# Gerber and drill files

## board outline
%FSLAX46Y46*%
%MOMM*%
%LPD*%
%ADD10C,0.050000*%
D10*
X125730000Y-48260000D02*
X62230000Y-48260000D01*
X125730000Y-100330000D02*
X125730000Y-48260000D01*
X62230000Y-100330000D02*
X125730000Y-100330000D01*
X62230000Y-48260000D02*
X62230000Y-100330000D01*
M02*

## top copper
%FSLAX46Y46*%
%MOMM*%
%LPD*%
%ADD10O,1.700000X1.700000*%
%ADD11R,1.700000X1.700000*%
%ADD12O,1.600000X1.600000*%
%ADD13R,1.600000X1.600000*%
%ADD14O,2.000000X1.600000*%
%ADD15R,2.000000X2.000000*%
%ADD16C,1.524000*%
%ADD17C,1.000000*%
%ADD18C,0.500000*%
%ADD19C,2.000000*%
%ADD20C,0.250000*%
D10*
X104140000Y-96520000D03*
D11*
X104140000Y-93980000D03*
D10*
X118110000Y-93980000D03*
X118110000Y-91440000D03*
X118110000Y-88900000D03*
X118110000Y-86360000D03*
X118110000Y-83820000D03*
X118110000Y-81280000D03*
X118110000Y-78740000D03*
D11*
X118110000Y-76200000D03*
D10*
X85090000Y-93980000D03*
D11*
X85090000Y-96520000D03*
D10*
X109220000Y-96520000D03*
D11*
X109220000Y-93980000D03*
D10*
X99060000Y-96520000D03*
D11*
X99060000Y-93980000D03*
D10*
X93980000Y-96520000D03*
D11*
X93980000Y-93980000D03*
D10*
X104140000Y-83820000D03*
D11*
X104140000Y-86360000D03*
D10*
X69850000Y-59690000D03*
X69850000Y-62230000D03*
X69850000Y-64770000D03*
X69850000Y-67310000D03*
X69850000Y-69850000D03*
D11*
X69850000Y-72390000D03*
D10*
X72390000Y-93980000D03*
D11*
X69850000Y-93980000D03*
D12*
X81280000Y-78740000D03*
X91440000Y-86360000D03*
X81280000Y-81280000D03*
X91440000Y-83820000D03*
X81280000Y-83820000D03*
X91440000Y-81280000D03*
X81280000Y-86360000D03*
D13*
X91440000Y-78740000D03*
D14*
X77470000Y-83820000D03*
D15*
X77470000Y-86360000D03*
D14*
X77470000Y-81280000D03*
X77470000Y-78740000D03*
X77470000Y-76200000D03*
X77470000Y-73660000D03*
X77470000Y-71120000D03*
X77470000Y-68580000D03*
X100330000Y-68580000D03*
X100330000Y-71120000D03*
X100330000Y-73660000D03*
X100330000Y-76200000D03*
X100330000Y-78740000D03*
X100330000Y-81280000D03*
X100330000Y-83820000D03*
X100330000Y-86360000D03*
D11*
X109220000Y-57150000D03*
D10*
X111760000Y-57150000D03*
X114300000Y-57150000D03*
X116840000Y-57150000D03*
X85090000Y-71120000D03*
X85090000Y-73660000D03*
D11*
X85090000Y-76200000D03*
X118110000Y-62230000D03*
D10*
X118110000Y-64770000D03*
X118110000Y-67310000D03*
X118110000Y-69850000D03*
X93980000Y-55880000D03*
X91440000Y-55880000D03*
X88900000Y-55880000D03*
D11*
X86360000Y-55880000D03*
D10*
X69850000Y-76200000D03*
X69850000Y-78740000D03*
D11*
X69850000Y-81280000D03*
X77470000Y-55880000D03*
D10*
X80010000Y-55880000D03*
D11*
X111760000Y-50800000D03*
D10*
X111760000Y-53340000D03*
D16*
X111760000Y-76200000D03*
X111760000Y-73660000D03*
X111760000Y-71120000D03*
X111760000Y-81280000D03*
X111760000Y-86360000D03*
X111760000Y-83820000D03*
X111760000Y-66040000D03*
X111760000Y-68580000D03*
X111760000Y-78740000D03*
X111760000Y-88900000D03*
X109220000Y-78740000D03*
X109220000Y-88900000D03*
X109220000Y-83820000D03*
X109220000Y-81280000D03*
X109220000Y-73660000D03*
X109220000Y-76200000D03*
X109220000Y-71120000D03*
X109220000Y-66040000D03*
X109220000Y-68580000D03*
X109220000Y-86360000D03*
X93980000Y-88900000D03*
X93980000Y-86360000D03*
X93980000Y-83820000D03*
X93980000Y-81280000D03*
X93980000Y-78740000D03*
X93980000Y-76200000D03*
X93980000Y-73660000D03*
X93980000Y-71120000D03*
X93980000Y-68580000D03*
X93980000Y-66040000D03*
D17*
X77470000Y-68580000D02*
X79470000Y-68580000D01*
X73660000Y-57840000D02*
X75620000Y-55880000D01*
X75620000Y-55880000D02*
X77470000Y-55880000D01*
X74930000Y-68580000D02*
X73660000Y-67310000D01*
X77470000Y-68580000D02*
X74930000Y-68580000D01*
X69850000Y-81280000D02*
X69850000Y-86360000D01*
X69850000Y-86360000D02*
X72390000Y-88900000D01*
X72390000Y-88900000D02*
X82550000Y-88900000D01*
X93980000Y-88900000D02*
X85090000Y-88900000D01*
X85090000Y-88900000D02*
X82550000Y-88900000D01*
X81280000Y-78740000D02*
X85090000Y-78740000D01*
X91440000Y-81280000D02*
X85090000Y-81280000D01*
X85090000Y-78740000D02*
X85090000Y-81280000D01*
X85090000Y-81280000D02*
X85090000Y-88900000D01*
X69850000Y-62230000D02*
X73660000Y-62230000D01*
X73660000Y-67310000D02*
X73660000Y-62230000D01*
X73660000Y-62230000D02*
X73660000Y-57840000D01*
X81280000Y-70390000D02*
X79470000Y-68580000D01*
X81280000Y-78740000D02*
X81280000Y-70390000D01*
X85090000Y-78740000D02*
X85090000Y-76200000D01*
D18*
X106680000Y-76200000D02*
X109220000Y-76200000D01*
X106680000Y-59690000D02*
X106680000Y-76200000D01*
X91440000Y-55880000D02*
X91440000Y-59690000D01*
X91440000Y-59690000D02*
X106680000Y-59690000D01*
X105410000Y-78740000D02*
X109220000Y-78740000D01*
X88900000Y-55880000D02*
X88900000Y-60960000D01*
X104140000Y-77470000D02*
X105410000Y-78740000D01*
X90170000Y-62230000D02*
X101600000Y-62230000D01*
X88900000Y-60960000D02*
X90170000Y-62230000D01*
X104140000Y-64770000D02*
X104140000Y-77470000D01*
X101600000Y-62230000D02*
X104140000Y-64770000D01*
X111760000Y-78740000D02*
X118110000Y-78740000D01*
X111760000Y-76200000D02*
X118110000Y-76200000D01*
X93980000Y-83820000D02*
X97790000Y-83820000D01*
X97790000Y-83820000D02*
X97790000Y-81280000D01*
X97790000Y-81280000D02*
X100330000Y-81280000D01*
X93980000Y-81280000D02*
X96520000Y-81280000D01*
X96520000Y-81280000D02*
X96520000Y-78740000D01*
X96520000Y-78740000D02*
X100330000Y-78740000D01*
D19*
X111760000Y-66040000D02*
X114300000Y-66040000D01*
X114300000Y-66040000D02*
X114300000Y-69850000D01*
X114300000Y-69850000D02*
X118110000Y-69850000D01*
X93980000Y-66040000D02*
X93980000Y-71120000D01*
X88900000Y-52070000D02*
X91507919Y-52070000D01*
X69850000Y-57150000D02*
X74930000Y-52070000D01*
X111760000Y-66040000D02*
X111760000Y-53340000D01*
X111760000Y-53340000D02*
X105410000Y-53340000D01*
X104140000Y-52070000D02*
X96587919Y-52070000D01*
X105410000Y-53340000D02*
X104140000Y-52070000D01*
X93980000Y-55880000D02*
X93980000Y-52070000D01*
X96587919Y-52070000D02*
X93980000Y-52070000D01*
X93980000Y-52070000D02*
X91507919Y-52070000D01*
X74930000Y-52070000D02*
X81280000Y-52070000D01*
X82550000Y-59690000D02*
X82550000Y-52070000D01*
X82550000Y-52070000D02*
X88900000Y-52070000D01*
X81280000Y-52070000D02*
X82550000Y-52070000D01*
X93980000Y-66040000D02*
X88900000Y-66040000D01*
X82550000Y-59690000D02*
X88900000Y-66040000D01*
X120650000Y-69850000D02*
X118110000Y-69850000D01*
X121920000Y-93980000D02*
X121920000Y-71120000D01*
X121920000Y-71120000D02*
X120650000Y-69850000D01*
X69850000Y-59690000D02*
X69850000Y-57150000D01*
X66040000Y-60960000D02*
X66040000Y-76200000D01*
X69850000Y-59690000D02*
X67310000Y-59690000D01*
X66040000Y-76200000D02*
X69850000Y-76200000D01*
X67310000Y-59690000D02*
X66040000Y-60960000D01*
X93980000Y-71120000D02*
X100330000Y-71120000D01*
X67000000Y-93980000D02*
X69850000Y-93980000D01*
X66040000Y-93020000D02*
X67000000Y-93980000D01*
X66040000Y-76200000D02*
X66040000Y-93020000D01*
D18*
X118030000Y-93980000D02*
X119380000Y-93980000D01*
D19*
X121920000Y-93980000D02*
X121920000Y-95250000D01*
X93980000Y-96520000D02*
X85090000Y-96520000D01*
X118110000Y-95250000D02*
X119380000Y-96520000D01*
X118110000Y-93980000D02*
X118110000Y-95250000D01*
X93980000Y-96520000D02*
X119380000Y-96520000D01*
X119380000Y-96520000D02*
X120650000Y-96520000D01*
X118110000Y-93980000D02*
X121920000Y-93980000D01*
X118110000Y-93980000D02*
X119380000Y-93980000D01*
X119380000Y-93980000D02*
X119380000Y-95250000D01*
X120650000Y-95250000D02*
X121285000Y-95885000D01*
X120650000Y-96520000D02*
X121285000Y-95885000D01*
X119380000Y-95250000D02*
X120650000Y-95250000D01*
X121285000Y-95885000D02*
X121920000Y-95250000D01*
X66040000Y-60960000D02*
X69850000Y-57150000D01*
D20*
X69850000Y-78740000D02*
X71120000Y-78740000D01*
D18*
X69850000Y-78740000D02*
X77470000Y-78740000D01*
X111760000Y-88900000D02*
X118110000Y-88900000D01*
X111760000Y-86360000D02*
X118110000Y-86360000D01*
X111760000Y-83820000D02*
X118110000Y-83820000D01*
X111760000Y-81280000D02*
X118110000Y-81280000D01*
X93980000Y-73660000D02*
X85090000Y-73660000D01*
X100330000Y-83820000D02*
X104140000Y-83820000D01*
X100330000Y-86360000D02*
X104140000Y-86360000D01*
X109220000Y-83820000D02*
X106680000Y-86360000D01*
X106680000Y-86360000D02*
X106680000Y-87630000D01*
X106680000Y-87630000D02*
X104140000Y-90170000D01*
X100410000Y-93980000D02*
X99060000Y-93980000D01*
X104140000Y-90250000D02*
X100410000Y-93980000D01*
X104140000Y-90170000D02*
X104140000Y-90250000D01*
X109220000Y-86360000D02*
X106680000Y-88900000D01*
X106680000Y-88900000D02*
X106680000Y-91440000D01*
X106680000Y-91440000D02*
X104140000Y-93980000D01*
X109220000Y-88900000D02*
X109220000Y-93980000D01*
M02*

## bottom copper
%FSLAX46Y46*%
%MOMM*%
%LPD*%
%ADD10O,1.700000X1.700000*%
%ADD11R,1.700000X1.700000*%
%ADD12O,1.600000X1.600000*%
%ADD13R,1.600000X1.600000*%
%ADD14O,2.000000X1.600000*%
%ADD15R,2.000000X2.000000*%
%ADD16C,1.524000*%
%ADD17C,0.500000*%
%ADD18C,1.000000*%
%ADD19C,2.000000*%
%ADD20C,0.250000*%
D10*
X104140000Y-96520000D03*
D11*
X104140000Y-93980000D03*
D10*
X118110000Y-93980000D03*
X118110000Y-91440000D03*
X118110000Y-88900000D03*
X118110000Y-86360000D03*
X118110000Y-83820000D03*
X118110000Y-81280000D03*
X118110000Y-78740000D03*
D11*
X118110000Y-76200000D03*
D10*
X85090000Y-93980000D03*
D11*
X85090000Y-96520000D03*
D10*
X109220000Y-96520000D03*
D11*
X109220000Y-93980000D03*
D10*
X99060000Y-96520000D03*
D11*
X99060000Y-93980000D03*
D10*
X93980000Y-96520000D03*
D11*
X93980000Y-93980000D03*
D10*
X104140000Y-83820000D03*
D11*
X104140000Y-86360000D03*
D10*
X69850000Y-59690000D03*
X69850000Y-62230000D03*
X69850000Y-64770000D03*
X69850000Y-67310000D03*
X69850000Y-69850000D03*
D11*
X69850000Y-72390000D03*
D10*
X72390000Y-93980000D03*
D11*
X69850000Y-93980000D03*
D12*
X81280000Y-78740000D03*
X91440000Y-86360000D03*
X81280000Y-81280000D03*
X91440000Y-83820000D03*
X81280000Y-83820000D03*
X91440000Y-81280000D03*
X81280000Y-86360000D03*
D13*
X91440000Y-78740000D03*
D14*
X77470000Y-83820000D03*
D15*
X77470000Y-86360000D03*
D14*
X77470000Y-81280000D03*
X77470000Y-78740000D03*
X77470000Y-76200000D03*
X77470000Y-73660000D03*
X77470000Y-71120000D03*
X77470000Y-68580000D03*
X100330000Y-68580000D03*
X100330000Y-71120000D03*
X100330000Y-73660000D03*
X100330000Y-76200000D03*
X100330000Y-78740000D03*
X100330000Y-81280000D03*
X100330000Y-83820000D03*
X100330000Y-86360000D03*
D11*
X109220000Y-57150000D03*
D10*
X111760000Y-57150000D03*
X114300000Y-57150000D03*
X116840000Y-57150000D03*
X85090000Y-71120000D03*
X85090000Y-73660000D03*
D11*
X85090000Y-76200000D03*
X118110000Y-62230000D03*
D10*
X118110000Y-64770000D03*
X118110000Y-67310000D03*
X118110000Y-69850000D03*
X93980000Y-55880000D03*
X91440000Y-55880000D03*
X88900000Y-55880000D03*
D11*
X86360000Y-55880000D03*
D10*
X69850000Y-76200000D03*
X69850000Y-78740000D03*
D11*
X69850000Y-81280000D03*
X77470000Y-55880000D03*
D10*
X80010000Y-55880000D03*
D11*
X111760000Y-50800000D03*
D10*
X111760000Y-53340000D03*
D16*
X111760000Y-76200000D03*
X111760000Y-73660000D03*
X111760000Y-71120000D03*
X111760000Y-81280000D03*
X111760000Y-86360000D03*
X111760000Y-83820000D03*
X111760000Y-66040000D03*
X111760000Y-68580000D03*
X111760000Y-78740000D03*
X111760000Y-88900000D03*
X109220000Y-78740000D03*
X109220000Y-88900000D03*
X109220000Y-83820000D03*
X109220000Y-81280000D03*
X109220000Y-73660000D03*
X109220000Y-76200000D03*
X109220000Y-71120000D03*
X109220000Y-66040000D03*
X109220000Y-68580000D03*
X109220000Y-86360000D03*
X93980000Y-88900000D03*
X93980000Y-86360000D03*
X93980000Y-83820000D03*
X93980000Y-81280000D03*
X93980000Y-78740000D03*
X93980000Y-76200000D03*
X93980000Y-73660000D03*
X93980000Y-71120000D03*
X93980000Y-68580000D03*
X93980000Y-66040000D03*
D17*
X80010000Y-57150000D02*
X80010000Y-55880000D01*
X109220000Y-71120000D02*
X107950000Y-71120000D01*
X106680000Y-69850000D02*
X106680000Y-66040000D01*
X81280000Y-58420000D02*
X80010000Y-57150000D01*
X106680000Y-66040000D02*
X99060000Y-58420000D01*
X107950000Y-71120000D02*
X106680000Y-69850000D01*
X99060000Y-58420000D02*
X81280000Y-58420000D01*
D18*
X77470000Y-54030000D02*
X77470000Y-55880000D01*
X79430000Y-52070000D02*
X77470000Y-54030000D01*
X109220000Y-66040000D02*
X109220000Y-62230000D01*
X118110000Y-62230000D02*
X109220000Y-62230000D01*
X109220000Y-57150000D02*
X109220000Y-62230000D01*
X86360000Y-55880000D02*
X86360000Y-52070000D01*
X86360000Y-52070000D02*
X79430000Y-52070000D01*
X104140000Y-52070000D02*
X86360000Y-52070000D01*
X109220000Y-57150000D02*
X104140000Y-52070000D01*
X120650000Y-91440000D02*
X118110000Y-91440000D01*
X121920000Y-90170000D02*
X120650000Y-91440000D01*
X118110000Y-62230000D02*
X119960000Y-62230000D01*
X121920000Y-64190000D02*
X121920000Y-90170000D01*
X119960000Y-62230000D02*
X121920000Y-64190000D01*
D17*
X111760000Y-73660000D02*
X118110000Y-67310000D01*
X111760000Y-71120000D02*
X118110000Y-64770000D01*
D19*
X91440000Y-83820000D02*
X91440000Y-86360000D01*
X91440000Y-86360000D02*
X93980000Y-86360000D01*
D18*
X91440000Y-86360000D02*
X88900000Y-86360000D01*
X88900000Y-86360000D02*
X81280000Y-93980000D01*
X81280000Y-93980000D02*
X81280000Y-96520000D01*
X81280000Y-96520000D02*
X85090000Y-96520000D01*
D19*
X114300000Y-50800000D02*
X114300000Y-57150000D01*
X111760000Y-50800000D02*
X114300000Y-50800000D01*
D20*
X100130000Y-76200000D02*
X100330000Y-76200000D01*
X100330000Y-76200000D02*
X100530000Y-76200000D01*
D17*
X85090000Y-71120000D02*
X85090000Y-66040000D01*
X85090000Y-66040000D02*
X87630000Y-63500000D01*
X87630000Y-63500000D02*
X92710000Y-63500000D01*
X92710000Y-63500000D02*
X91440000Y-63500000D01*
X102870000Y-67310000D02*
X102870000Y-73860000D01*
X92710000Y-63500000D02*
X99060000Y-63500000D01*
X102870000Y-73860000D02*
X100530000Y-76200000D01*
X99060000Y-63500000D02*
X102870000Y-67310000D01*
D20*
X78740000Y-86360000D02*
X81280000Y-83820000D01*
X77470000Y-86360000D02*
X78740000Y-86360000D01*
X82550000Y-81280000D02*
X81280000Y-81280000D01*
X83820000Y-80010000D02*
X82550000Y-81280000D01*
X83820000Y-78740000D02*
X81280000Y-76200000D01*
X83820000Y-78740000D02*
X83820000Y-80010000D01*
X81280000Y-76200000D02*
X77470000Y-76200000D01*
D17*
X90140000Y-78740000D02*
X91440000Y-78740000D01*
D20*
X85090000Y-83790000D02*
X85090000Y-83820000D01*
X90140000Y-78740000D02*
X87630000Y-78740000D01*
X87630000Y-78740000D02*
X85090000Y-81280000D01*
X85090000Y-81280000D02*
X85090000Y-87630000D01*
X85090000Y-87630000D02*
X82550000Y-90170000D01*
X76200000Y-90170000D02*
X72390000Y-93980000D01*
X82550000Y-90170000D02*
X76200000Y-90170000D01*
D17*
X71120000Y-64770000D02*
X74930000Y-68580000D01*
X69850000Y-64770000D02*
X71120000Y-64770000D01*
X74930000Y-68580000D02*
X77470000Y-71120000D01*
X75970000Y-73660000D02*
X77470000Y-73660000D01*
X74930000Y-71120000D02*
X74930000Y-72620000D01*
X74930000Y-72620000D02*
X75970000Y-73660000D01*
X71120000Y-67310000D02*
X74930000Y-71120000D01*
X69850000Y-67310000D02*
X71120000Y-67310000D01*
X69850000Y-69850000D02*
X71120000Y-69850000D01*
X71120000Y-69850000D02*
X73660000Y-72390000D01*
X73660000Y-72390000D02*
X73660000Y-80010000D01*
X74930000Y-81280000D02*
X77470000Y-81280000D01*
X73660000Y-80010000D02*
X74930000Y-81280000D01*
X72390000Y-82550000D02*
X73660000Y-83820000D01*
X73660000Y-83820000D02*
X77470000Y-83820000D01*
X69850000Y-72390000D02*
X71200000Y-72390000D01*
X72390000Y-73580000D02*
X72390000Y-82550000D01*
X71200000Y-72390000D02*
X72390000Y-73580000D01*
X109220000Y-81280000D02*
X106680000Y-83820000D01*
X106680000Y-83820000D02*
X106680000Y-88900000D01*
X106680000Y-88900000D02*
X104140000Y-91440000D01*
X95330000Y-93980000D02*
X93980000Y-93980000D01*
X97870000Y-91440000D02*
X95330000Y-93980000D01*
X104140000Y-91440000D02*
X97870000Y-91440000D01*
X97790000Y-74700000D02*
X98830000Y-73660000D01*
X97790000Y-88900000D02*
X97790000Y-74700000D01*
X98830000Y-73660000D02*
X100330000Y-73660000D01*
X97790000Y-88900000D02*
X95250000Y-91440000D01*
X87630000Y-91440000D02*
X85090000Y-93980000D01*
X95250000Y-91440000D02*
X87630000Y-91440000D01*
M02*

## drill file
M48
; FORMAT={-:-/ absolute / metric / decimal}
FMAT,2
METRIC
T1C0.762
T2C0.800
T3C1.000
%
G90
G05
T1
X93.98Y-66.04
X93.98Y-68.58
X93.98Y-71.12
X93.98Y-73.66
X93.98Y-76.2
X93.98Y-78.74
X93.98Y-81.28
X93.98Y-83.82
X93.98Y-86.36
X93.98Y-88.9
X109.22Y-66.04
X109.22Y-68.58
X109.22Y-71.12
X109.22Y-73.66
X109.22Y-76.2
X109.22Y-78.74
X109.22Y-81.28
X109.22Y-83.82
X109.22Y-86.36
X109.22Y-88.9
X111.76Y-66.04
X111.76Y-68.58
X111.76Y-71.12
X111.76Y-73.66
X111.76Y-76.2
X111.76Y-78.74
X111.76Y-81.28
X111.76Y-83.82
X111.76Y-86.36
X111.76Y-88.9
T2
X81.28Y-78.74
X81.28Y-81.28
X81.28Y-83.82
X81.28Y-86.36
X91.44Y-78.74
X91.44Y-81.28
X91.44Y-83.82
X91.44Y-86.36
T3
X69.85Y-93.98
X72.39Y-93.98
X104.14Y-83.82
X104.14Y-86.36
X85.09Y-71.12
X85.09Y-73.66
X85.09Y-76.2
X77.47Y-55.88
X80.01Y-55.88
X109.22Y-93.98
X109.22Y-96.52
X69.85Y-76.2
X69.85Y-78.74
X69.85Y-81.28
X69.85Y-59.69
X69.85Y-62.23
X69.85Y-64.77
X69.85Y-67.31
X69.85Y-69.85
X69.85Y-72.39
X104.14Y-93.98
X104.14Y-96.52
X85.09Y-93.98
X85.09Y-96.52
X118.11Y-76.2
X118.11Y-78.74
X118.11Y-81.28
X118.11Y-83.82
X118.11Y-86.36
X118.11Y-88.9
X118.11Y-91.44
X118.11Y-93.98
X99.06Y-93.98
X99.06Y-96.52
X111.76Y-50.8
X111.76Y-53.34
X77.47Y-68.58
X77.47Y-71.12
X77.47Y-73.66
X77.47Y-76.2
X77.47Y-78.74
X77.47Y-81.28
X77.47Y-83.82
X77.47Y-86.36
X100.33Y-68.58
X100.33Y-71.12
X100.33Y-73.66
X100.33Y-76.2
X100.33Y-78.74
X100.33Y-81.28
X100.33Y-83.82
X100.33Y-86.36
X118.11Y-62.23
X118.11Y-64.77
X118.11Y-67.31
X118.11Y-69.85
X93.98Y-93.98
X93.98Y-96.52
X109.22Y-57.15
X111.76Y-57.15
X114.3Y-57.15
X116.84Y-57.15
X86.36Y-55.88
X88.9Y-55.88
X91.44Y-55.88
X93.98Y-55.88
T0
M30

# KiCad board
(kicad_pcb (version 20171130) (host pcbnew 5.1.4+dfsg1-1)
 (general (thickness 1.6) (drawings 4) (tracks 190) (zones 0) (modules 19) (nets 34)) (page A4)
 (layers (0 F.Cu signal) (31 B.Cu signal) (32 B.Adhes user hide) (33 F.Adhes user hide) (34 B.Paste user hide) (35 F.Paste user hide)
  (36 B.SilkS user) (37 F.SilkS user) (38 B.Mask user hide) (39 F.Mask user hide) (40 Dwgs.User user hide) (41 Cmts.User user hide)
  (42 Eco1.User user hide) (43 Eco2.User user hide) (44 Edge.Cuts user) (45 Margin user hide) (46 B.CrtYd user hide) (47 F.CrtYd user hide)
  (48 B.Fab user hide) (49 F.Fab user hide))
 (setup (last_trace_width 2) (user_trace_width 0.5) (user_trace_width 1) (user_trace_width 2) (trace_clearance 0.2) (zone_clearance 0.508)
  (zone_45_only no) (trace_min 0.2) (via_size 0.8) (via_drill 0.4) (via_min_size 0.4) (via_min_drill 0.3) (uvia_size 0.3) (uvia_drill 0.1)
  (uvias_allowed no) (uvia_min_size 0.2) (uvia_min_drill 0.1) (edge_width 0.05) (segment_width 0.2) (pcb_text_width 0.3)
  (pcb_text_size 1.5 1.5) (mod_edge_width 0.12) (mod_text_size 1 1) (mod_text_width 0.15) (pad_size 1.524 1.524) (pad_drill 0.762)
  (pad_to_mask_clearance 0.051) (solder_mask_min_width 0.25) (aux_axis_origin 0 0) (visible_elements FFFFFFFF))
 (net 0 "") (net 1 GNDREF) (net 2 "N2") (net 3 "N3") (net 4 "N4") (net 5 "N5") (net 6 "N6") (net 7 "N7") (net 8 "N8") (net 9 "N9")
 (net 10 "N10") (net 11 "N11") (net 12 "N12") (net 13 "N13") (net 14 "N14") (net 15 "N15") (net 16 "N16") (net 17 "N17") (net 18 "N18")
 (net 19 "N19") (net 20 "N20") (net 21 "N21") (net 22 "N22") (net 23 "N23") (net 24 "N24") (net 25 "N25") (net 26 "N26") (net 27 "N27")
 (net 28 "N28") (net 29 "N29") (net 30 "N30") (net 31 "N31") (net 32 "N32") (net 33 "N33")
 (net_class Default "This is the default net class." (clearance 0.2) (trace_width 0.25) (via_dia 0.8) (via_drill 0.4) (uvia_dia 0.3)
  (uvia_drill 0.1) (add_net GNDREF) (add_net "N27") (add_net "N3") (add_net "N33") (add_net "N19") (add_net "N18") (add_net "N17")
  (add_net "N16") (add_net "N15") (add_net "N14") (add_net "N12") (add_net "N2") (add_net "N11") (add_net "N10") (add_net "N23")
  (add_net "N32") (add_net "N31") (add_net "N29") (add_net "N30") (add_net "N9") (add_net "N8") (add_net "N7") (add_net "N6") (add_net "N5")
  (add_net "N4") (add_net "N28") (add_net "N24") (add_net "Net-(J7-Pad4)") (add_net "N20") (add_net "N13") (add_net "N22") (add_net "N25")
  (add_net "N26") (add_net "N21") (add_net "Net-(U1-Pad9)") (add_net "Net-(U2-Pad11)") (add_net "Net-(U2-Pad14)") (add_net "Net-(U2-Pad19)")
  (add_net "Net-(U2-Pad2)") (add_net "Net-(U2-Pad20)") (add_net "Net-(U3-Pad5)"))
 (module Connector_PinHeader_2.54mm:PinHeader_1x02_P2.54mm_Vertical (layer F.Cu) (at 104.14 93.98)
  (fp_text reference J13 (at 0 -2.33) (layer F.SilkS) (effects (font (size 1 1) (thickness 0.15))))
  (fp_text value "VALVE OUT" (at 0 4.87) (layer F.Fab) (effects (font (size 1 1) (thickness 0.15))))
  (pad 2 thru_hole oval (at 0 2.54) (size 1.7 1.7) (drill 1) (layers *.Cu *.Mask) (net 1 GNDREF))
  (pad 1 thru_hole rect (at 0 0) (size 1.7 1.7) (drill 1) (layers *.Cu *.Mask) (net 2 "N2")))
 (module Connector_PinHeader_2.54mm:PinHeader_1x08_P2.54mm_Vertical (layer F.Cu) (at 118.11 76.2)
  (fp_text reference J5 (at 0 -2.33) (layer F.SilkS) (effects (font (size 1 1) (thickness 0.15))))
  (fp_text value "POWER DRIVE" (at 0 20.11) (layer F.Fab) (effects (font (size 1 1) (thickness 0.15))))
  (pad 8 thru_hole oval (at 0 17.78) (size 1.7 1.7) (drill 1) (layers *.Cu *.Mask) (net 1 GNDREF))
  (pad 7 thru_hole oval (at 0 15.24) (size 1.7 1.7) (drill 1) (layers *.Cu *.Mask) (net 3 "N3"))
  (pad 6 thru_hole oval (at 0 12.7) (size 1.7 1.7) (drill 1) (layers *.Cu *.Mask) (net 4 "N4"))
  (pad 5 thru_hole oval (at 0 10.16) (size 1.7 1.7) (drill 1) (layers *.Cu *.Mask) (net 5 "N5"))
  (pad 4 thru_hole oval (at 0 7.62) (size 1.7 1.7) (drill 1) (layers *.Cu *.Mask) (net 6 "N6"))
  (pad 3 thru_hole oval (at 0 5.08) (size 1.7 1.7) (drill 1) (layers *.Cu *.Mask) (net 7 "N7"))
  (pad 2 thru_hole oval (at 0 2.54) (size 1.7 1.7) (drill 1) (layers *.Cu *.Mask) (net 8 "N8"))
  (pad 1 thru_hole rect (at 0 0) (size 1.7 1.7) (drill 1) (layers *.Cu *.Mask) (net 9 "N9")))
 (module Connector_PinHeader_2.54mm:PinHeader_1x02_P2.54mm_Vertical (layer F.Cu) (at 85.09 96.52 180)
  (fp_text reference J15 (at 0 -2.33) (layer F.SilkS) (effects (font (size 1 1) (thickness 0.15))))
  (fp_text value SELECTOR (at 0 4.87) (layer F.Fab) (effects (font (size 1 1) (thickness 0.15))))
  (pad 2 thru_hole oval (at 0 2.54 180) (size 1.7 1.7) (drill 1) (layers *.Cu *.Mask) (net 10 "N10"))
  (pad 1 thru_hole rect (at 0 0 180) (size 1.7 1.7) (drill 1) (layers *.Cu *.Mask) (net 1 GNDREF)))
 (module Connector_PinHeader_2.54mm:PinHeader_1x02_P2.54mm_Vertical (layer F.Cu) (at 109.22 93.98)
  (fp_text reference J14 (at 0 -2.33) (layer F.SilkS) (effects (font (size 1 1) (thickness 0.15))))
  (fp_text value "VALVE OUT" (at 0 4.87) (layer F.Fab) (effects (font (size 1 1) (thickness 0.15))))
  (pad 2 thru_hole oval (at 0 2.54) (size 1.7 1.7) (drill 1) (layers *.Cu *.Mask) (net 1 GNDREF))
  (pad 1 thru_hole rect (at 0 0) (size 1.7 1.7) (drill 1) (layers *.Cu *.Mask) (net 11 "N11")))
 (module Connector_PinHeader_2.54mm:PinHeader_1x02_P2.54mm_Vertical (layer F.Cu) (at 99.06 93.98)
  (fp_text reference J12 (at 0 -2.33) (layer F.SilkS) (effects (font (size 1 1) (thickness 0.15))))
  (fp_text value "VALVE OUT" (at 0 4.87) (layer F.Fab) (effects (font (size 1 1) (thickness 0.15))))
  (pad 2 thru_hole oval (at 0 2.54) (size 1.7 1.7) (drill 1) (layers *.Cu *.Mask) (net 1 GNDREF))
  (pad 1 thru_hole rect (at 0 0) (size 1.7 1.7) (drill 1) (layers *.Cu *.Mask) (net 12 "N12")))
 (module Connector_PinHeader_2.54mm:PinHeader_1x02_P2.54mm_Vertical (layer F.Cu) (at 93.98 93.98)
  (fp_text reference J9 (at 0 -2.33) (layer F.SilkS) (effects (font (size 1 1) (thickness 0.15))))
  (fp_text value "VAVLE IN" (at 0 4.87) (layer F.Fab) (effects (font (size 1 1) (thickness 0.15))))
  (pad 2 thru_hole oval (at 0 2.54) (size 1.7 1.7) (drill 1) (layers *.Cu *.Mask) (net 1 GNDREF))
  (pad 1 thru_hole rect (at 0 0) (size 1.7 1.7) (drill 1) (layers *.Cu *.Mask) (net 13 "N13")))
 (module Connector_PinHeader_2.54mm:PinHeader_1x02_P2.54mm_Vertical (layer B.Cu) (at 104.14 86.36)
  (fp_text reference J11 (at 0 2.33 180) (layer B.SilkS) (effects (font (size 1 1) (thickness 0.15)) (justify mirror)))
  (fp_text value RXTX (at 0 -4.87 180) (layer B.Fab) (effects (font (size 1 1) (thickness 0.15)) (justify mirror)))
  (pad 2 thru_hole oval (at 0 -2.54) (size 1.7 1.7) (drill 1) (layers *.Cu *.Mask) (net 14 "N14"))
  (pad 1 thru_hole rect (at 0 0) (size 1.7 1.7) (drill 1) (layers *.Cu *.Mask) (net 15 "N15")))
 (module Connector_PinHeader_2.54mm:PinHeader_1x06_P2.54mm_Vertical (layer F.Cu) (at 69.85 72.39 180)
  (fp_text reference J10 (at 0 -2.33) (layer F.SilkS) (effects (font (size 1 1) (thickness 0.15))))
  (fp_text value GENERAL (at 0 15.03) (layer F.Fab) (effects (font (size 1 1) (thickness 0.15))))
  (pad 6 thru_hole oval (at 0 12.7 180) (size 1.7 1.7) (drill 1) (layers *.Cu *.Mask) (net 1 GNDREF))
  (pad 5 thru_hole oval (at 0 10.16 180) (size 1.7 1.7) (drill 1) (layers *.Cu *.Mask) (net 3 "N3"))
  (pad 4 thru_hole oval (at 0 7.62 180) (size 1.7 1.7) (drill 1) (layers *.Cu *.Mask) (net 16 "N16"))
  (pad 3 thru_hole oval (at 0 5.08 180) (size 1.7 1.7) (drill 1) (layers *.Cu *.Mask) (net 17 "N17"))
  (pad 2 thru_hole oval (at 0 2.54 180) (size 1.7 1.7) (drill 1) (layers *.Cu *.Mask) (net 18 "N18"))
  (pad 1 thru_hole rect (at 0 0 180) (size 1.7 1.7) (drill 1) (layers *.Cu *.Mask) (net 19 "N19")))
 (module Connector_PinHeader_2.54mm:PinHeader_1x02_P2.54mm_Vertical (layer F.Cu) (at 69.85 93.98 90)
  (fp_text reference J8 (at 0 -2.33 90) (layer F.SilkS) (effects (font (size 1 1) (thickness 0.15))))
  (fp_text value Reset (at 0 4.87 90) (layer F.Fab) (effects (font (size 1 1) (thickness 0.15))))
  (pad 2 thru_hole oval (at 0 2.54 90) (size 1.7 1.7) (drill 1) (layers *.Cu *.Mask) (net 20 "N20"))
  (pad 1 thru_hole rect (at 0 0 90) (size 1.7 1.7) (drill 1) (layers *.Cu *.Mask) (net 1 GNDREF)))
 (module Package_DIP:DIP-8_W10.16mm (layer B.Cu) (at 91.44 78.74 180)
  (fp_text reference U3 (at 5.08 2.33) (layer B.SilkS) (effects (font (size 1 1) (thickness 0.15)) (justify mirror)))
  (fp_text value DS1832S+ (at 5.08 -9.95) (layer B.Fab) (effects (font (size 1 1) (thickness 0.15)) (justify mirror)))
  (pad 8 thru_hole oval (at 10.16 0 180) (size 1.6 1.6) (drill 0.8) (layers *.Cu *.Mask) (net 3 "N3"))
  (pad 4 thru_hole oval (at 0 -7.62 180) (size 1.6 1.6) (drill 0.8) (layers *.Cu *.Mask) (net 1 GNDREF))
  (pad 7 thru_hole oval (at 10.16 -2.54 180) (size 1.6 1.6) (drill 0.8) (layers *.Cu *.Mask) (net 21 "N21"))
  (pad 3 thru_hole oval (at 0 -5.08 180) (size 1.6 1.6) (drill 0.8) (layers *.Cu *.Mask) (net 1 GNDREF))
  (pad 6 thru_hole oval (at 10.16 -5.08 180) (size 1.6 1.6) (drill 0.8) (layers *.Cu *.Mask) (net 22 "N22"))
  (pad 2 thru_hole oval (at 0 -2.54 180) (size 1.6 1.6) (drill 0.8) (layers *.Cu *.Mask) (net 3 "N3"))
  (pad 5 thru_hole oval (at 10.16 -7.62 180) (size 1.6 1.6) (drill 0.8) (layers *.Cu *.Mask))
  (pad 1 thru_hole rect (at 0 0 180) (size 1.6 1.6) (drill 0.8) (layers *.Cu *.Mask) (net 20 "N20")))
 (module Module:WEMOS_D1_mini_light (layer B.Cu) (at 77.47 86.36)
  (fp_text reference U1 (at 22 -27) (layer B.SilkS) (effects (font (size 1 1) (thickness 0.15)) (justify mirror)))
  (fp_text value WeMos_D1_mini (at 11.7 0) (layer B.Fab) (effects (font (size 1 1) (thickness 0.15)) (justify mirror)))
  (pad 2 thru_hole oval (at 0 -2.54) (size 2 1.6) (drill 1) (layers *.Cu *.Mask) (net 19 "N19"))
  (pad 1 thru_hole rect (at 0 0) (size 2 2) (drill 1) (layers *.Cu *.Mask) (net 22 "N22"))
  (pad 3 thru_hole oval (at 0 -5.08) (size 2 1.6) (drill 1) (layers *.Cu *.Mask) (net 18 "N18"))
  (pad 4 thru_hole oval (at 0 -7.62) (size 2 1.6) (drill 1) (layers *.Cu *.Mask) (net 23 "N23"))
  (pad 5 thru_hole oval (at 0 -10.16) (size 2 1.6) (drill 1) (layers *.Cu *.Mask) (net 21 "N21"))
  (pad 6 thru_hole oval (at 0 -12.7) (size 2 1.6) (drill 1) (layers *.Cu *.Mask) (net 17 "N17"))
  (pad 7 thru_hole oval (at 0 -15.24) (size 2 1.6) (drill 1) (layers *.Cu *.Mask) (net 16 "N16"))
  (pad 8 thru_hole oval (at 0 -17.78) (size 2 1.6) (drill 1) (layers *.Cu *.Mask) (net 3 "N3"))
  (pad 9 thru_hole oval (at 22.86 -17.78) (size 2 1.6) (drill 1) (layers *.Cu *.Mask))
  (pad 10 thru_hole oval (at 22.86 -15.24) (size 2 1.6) (drill 1) (layers *.Cu *.Mask) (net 1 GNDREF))
  (pad 11 thru_hole oval (at 22.86 -12.7) (size 2 1.6) (drill 1) (layers *.Cu *.Mask) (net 10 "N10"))
  (pad 12 thru_hole oval (at 22.86 -10.16) (size 2 1.6) (drill 1) (layers *.Cu *.Mask) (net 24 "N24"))
  (pad 13 thru_hole oval (at 22.86 -7.62) (size 2 1.6) (drill 1) (layers *.Cu *.Mask) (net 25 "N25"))
  (pad 14 thru_hole oval (at 22.86 -5.08) (size 2 1.6) (drill 1) (layers *.Cu *.Mask) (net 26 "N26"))
  (pad 15 thru_hole oval (at 22.86 -2.54) (size 2 1.6) (drill 1) (layers *.Cu *.Mask) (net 14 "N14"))
  (pad 16 thru_hole oval (at 22.86 0) (size 2 1.6) (drill 1) (layers *.Cu *.Mask) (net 15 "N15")))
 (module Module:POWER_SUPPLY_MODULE (layer B.Cu) (at 109.22 57.15 270)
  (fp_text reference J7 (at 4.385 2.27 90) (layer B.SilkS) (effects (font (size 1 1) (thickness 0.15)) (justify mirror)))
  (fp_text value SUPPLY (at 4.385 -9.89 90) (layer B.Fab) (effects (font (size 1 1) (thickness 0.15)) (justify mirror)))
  (pad 1 thru_hole rect (at 0 0 270) (size 1.7 1.7) (drill 1) (layers *.Cu *.Mask) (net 3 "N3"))
  (pad 2 thru_hole oval (at 0 -2.54 270) (size 1.7 1.7) (drill 1) (layers *.Cu *.Mask) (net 1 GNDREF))
  (pad 3 thru_hole oval (at 0 -5.08 270) (size 1.7 1.7) (drill 1) (layers *.Cu *.Mask) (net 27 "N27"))
  (pad 4 thru_hole oval (at 0 -7.62 270) (size 1.7 1.7) (drill 1) (layers *.Cu *.Mask)))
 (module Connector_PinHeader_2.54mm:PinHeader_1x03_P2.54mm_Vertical (layer F.Cu) (at 85.09 76.2 180)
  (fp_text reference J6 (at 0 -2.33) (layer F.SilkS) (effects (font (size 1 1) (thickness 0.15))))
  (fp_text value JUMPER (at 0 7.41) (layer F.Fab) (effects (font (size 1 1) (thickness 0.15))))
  (pad 3 thru_hole oval (at 0 5.08 180) (size 1.7 1.7) (drill 1) (layers *.Cu *.Mask) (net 24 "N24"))
  (pad 2 thru_hole oval (at 0 2.54 180) (size 1.7 1.7) (drill 1) (layers *.Cu *.Mask) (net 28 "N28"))
  (pad 1 thru_hole rect (at 0 0 180) (size 1.7 1.7) (drill 1) (layers *.Cu *.Mask) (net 3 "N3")))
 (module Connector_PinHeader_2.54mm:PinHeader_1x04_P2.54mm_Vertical (layer F.Cu) (at 118.11 62.23)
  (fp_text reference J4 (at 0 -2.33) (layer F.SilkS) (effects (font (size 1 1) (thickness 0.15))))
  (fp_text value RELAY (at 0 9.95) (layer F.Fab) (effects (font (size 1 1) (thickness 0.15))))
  (pad 1 thru_hole rect (at 0 0) (size 1.7 1.7) (drill 1) (layers *.Cu *.Mask) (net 3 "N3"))
  (pad 2 thru_hole oval (at 0 2.54) (size 1.7 1.7) (drill 1) (layers *.Cu *.Mask) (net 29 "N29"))
  (pad 3 thru_hole oval (at 0 5.08) (size 1.7 1.7) (drill 1) (layers *.Cu *.Mask) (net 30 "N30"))
  (pad 4 thru_hole oval (at 0 7.62) (size 1.7 1.7) (drill 1) (layers *.Cu *.Mask) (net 1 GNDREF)))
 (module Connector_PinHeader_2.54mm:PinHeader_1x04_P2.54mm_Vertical (layer F.Cu) (at 86.36 55.88 90)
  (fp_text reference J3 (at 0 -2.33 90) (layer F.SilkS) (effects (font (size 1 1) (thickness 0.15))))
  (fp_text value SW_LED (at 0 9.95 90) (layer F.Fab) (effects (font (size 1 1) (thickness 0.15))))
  (pad 4 thru_hole oval (at 0 7.62 90) (size 1.7 1.7) (drill 1) (layers *.Cu *.Mask) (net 1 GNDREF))
  (pad 3 thru_hole oval (at 0 5.08 90) (size 1.7 1.7) (drill 1) (layers *.Cu *.Mask) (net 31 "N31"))
  (pad 2 thru_hole oval (at 0 2.54 90) (size 1.7 1.7) (drill 1) (layers *.Cu *.Mask) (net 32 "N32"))
  (pad 1 thru_hole rect (at 0 0 90) (size 1.7 1.7) (drill 1) (layers *.Cu *.Mask) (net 3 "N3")))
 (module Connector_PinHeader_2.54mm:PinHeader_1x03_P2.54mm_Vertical (layer F.Cu) (at 69.85 81.28 180)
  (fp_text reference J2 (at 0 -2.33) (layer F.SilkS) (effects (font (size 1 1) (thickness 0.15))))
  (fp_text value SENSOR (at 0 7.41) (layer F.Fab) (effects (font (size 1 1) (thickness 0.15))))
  (pad 3 thru_hole oval (at 0 5.08 180) (size 1.7 1.7) (drill 1) (layers *.Cu *.Mask) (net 1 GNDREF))
  (pad 2 thru_hole oval (at 0 2.54 180) (size 1.7 1.7) (drill 1) (layers *.Cu *.Mask) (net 23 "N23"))
  (pad 1 thru_hole rect (at 0 0 180) (size 1.7 1.7) (drill 1) (layers *.Cu *.Mask) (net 3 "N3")))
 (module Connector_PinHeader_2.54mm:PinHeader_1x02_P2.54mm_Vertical (layer F.Cu) (at 77.47 55.88 90)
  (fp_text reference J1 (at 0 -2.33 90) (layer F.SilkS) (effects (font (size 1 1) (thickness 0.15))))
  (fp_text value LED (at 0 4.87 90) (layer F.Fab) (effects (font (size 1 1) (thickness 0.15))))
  (pad 1 thru_hole rect (at 0 0 90) (size 1.7 1.7) (drill 1) (layers *.Cu *.Mask) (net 3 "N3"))
  (pad 2 thru_hole oval (at 0 2.54 90) (size 1.7 1.7) (drill 1) (layers *.Cu *.Mask) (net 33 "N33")))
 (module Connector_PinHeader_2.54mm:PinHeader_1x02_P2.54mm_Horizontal (layer F.Cu) (at 111.76 50.8)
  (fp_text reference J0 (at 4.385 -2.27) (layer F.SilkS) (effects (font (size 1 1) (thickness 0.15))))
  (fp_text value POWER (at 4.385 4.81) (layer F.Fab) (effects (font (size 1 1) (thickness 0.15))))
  (pad 1 thru_hole rect (at 0 0) (size 1.7 1.7) (drill 1) (layers *.Cu *.Mask) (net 27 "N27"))
  (pad 2 thru_hole oval (at 0 2.54) (size 1.7 1.7) (drill 1) (layers *.Cu *.Mask) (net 1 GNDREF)))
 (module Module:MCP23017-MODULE (layer F.Cu) (at 102.87 62.23)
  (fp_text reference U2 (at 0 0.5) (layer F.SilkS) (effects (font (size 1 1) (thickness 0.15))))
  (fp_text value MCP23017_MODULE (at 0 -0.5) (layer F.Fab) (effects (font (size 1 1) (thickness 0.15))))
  (pad 23 thru_hole circle (at 8.89 13.97) (size 1.524 1.524) (drill 0.762) (layers *.Cu *.Mask) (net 9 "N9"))
  (pad 22 thru_hole circle (at 8.89 11.43) (size 1.524 1.524) (drill 0.762) (layers *.Cu *.Mask) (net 30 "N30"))
  (pad 21 thru_hole circle (at 8.89 8.89) (size 1.524 1.524) (drill 0.762) (layers *.Cu *.Mask) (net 29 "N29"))
  (pad 25 thru_hole circle (at 8.89 19.05) (size 1.524 1.524) (drill 0.762) (layers *.Cu *.Mask) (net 7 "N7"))
  (pad 27 thru_hole circle (at 8.89 24.13) (size 1.524 1.524) (drill 0.762) (layers *.Cu *.Mask) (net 5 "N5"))
  (pad 26 thru_hole circle (at 8.89 21.59) (size 1.524 1.524) (drill 0.762) (layers *.Cu *.Mask) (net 6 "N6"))
  (pad 30 thru_hole circle (at 8.89 3.81) (size 1.524 1.524) (drill 0.762) (layers *.Cu *.Mask) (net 1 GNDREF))
  (pad 20 thru_hole circle (at 8.89 6.35) (size 1.524 1.524) (drill 0.762) (layers *.Cu *.Mask))
  (pad 24 thru_hole circle (at 8.89 16.51) (size 1.524 1.524) (drill 0.762) (layers *.Cu *.Mask) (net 8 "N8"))
  (pad 28 thru_hole circle (at 8.89 26.67) (size 1.524 1.524) (drill 0.762) (layers *.Cu *.Mask) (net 4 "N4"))
  (pad 4 thru_hole circle (at 6.35 16.51) (size 1.524 1.524) (drill 0.762) (layers *.Cu *.Mask) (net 32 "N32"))
  (pad 8 thru_hole circle (at 6.35 26.67) (size 1.524 1.524) (drill 0.762) (layers *.Cu *.Mask) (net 11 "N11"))
  (pad 6 thru_hole circle (at 6.35 21.59) (size 1.524 1.524) (drill 0.762) (layers *.Cu *.Mask) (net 12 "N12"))
  (pad 5 thru_hole circle (at 6.35 19.05) (size 1.524 1.524) (drill 0.762) (layers *.Cu *.Mask) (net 13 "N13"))
  (pad 2 thru_hole circle (at 6.35 11.43) (size 1.524 1.524) (drill 0.762) (layers *.Cu *.Mask))
  (pad 3 thru_hole circle (at 6.35 13.97) (size 1.524 1.524) (drill 0.762) (layers *.Cu *.Mask) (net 31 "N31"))
  (pad 1 thru_hole circle (at 6.35 8.89) (size 1.524 1.524) (drill 0.762) (layers *.Cu *.Mask) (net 33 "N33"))
  (pad 29 thru_hole circle (at 6.35 3.81) (size 1.524 1.524) (drill 0.762) (layers *.Cu *.Mask) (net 3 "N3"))
  (pad 19 thru_hole circle (at 6.35 6.35) (size 1.524 1.524) (drill 0.762) (layers *.Cu *.Mask))
  (pad 7 thru_hole circle (at 6.35 24.13) (size 1.524 1.524) (drill 0.762) (layers *.Cu *.Mask) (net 2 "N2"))
  (pad 9 thru_hole circle (at -8.89 26.67) (size 1.524 1.524) (drill 0.762) (layers *.Cu *.Mask) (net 3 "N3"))
  (pad 10 thru_hole circle (at -8.89 24.13) (size 1.524 1.524) (drill 0.762) (layers *.Cu *.Mask) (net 1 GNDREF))
  (pad 12 thru_hole circle (at -8.89 21.59) (size 1.524 1.524) (drill 0.762) (layers *.Cu *.Mask) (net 26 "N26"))
  (pad 13 thru_hole circle (at -8.89 19.05) (size 1.524 1.524) (drill 0.762) (layers *.Cu *.Mask) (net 25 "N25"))
  (pad 14 thru_hole circle (at -8.89 16.51) (size 1.524 1.524) (drill 0.762) (layers *.Cu *.Mask))
  (pad 11 thru_hole circle (at -8.89 13.97) (size 1.524 1.524) (drill 0.762) (layers *.Cu *.Mask))
  (pad 18 thru_hole circle (at -8.89 11.43) (size 1.524 1.524) (drill 0.762) (layers *.Cu *.Mask) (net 28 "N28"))
  (pad 15 thru_hole circle (at -8.89 8.89) (size 1.524 1.524) (drill 0.762) (layers *.Cu *.Mask) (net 1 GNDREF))
  (pad 16 thru_hole circle (at -8.89 6.35) (size 1.524 1.524) (drill 0.762) (layers *.Cu *.Mask) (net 1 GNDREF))
  (pad 17 thru_hole circle (at -8.89 3.81) (size 1.524 1.524) (drill 0.762) (layers *.Cu *.Mask) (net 1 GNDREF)))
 (gr_line (start 125.73 48.26) (end 62.23 48.26) (layer Edge.Cuts) (width 0.05))
 (gr_line (start 125.73 100.33) (end 125.73 48.26) (layer Edge.Cuts) (width 0.05))
 (gr_line (start 62.23 100.33) (end 125.73 100.33) (layer Edge.Cuts) (width 0.05))
 (gr_line (start 62.23 48.26) (end 62.23 100.33) (layer Edge.Cuts) (width 0.05))
 (segment (start 80.01 57.15) (end 80.01 55.88) (width 0.5) (layer B.Cu) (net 33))
 (segment (start 109.22 71.12) (end 107.95 71.12) (width 0.5) (layer B.Cu) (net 33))
 (segment (start 106.68 69.85) (end 106.68 66.04) (width 0.5) (layer B.Cu) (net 33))
 (segment (start 81.28 58.42) (end 80.01 57.15) (width 0.5) (layer B.Cu) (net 33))
 (segment (start 106.68 66.04) (end 99.06 58.42) (width 0.5) (layer B.Cu) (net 33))
 (segment (start 107.95 71.12) (end 106.68 69.85) (width 0.5) (layer B.Cu) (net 33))
 (segment (start 99.06 58.42) (end 81.28 58.42) (width 0.5) (layer B.Cu) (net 33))
 (segment (start 77.47 68.58) (end 79.47 68.58) (width 1) (layer F.Cu) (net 3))
 (segment (start 73.66 57.84) (end 75.62 55.88) (width 1) (layer F.Cu) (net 3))
 (segment (start 75.62 55.88) (end 77.47 55.88) (width 1) (layer F.Cu) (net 3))
 (segment (start 74.93 68.58) (end 73.66 67.31) (width 1) (layer F.Cu) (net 3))
 (segment (start 77.47 68.58) (end 74.93 68.58) (width 1) (layer F.Cu) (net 3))
 (segment (start 77.47 54.03) (end 77.47 55.88) (width 1) (layer B.Cu) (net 3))
 (segment (start 79.43 52.07) (end 77.47 54.03) (width 1) (layer B.Cu) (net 3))
 (segment (start 109.22 66.04) (end 109.22 62.23) (width 1) (layer B.Cu) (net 3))
 (segment (start 118.11 62.23) (end 109.22 62.23) (width 1) (layer B.Cu) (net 3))
 (segment (start 69.85 81.28) (end 69.85 86.36) (width 1) (layer F.Cu) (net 3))
 (segment (start 69.85 86.36) (end 72.39 88.9) (width 1) (layer F.Cu) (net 3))
 (segment (start 72.39 88.9) (end 82.55 88.9) (width 1) (layer F.Cu) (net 3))
 (segment (start 109.22 57.15) (end 109.22 62.23) (width 1) (layer B.Cu) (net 3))
 (segment (start 86.36 55.88) (end 86.36 52.07) (width 1) (layer B.Cu) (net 3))
 (segment (start 86.36 52.07) (end 79.43 52.07) (width 1) (layer B.Cu) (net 3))
 (segment (start 93.98 88.9) (end 85.09 88.9) (width 1) (layer F.Cu) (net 3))
 (segment (start 85.09 88.9) (end 82.55 88.9) (width 1) (layer F.Cu) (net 3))
 (segment (start 81.28 78.74) (end 85.09 78.74) (width 1) (layer F.Cu) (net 3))
 (segment (start 91.44 81.28) (end 85.09 81.28) (width 1) (layer F.Cu) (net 3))
 (segment (start 85.09 78.74) (end 85.09 81.28) (width 1) (layer F.Cu) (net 3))
 (segment (start 85.09 81.28) (end 85.09 88.9) (width 1) (layer F.Cu) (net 3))
 (segment (start 104.14 52.07) (end 86.36 52.07) (width 1) (layer B.Cu) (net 3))
 (segment (start 109.22 57.15) (end 104.14 52.07) (width 1) (layer B.Cu) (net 3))
 (segment (start 69.85 62.23) (end 73.66 62.23) (width 1) (layer F.Cu) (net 3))
 (segment (start 73.66 67.31) (end 73.66 62.23) (width 1) (layer F.Cu) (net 3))
 (segment (start 73.66 62.23) (end 73.66 57.84) (width 1) (layer F.Cu) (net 3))
 (segment (start 81.28 70.39) (end 79.47 68.58) (width 1) (layer F.Cu) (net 3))
 (segment (start 81.28 78.74) (end 81.28 70.39) (width 1) (layer F.Cu) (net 3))
 (segment (start 85.09 78.74) (end 85.09 76.2) (width 1) (layer F.Cu) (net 3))
 (segment (start 120.65 91.44) (end 118.11 91.44) (width 1) (layer B.Cu) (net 3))
 (segment (start 121.92 90.17) (end 120.65 91.44) (width 1) (layer B.Cu) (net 3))
 (segment (start 118.11 62.23) (end 119.96 62.23) (width 1) (layer B.Cu) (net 3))
 (segment (start 121.92 64.19) (end 121.92 90.17) (width 1) (layer B.Cu) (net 3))
 (segment (start 119.96 62.23) (end 121.92 64.19) (width 1) (layer B.Cu) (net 3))
 (segment (start 106.68 76.2) (end 109.22 76.2) (width 0.5) (layer F.Cu) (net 31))
 (segment (start 106.68 59.69) (end 106.68 76.2) (width 0.5) (layer F.Cu) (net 31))
 (segment (start 91.44 55.88) (end 91.44 59.69) (width 0.5) (layer F.Cu) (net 31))
 (segment (start 91.44 59.69) (end 106.68 59.69) (width 0.5) (layer F.Cu) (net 31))
 (segment (start 105.41 78.74) (end 109.22 78.74) (width 0.5) (layer F.Cu) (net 32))
 (segment (start 88.9 55.88) (end 88.9 60.96) (width 0.5) (layer F.Cu) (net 32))
 (segment (start 104.14 77.47) (end 105.41 78.74) (width 0.5) (layer F.Cu) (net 32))
 (segment (start 90.17 62.23) (end 101.6 62.23) (width 0.5) (layer F.Cu) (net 32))
 (segment (start 88.9 60.96) (end 90.17 62.23) (width 0.5) (layer F.Cu) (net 32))
 (segment (start 104.14 64.77) (end 104.14 77.47) (width 0.5) (layer F.Cu) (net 32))
 (segment (start 101.6 62.23) (end 104.14 64.77) (width 0.5) (layer F.Cu) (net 32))
 (segment (start 111.76 73.66) (end 118.11 67.31) (width 0.5) (layer B.Cu) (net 30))
 (segment (start 111.76 71.12) (end 118.11 64.77) (width 0.5) (layer B.Cu) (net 29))
 (segment (start 111.76 78.74) (end 118.11 78.74) (width 0.5) (layer F.Cu) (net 8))
 (segment (start 111.76 76.2) (end 118.11 76.2) (width 0.5) (layer F.Cu) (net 9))
 (segment (start 93.98 83.82) (end 97.79 83.82) (width 0.5) (layer F.Cu) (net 26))
 (segment (start 97.79 83.82) (end 97.79 81.28) (width 0.5) (layer F.Cu) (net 26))
 (segment (start 97.79 81.28) (end 100.33 81.28) (width 0.5) (layer F.Cu) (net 26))
 (segment (start 93.98 81.28) (end 96.52 81.28) (width 0.5) (layer F.Cu) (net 25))
 (segment (start 96.52 81.28) (end 96.52 78.74) (width 0.5) (layer F.Cu) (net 25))
 (segment (start 96.52 78.74) (end 100.33 78.74) (width 0.5) (layer F.Cu) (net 25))
 (segment (start 111.76 66.04) (end 114.3 66.04) (width 2) (layer F.Cu) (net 1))
 (segment (start 114.3 66.04) (end 114.3 69.85) (width 2) (layer F.Cu) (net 1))
 (segment (start 114.3 69.85) (end 118.11 69.85) (width 2) (layer F.Cu) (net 1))
 (segment (start 93.98 66.04) (end 93.98 71.12) (width 2) (layer F.Cu) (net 1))
 (segment (start 88.9 52.07) (end 91.507919 52.07) (width 2) (layer F.Cu) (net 1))
 (segment (start 69.85 57.15) (end 74.93 52.07) (width 2) (layer F.Cu) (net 1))
 (segment (start 111.76 66.04) (end 111.76 53.34) (width 2) (layer F.Cu) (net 1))
 (segment (start 111.76 53.34) (end 105.41 53.34) (width 2) (layer F.Cu) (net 1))
 (segment (start 104.14 52.07) (end 96.587919 52.07) (width 2) (layer F.Cu) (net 1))
 (segment (start 105.41 53.34) (end 104.14 52.07) (width 2) (layer F.Cu) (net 1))
 (segment (start 93.98 55.88) (end 93.98 52.07) (width 2) (layer F.Cu) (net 1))
 (segment (start 96.587919 52.07) (end 93.98 52.07) (width 2) (layer F.Cu) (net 1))
 (segment (start 93.98 52.07) (end 91.507919 52.07) (width 2) (layer F.Cu) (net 1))
 (segment (start 74.93 52.07) (end 81.28 52.07) (width 2) (layer F.Cu) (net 1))
 (segment (start 82.55 59.69) (end 82.55 52.07) (width 2) (layer F.Cu) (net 1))
 (segment (start 82.55 52.07) (end 88.9 52.07) (width 2) (layer F.Cu) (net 1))
 (segment (start 81.28 52.07) (end 82.55 52.07) (width 2) (layer F.Cu) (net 1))
 (segment (start 93.98 66.04) (end 88.9 66.04) (width 2) (layer F.Cu) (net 1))
 (segment (start 82.55 59.69) (end 88.9 66.04) (width 2) (layer F.Cu) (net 1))
 (segment (start 91.44 83.82) (end 91.44 86.36) (width 2) (layer B.Cu) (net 1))
 (segment (start 120.65 69.85) (end 118.11 69.85) (width 2) (layer F.Cu) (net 1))
 (segment (start 121.92 93.98) (end 121.92 71.12) (width 2) (layer F.Cu) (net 1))
 (segment (start 121.92 71.12) (end 120.65 69.85) (width 2) (layer F.Cu) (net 1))
 (segment (start 69.85 59.69) (end 69.85 57.15) (width 2) (layer F.Cu) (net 1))
 (segment (start 66.04 60.96) (end 66.04 76.2) (width 2) (layer F.Cu) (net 1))
 (segment (start 69.85 59.69) (end 67.31 59.69) (width 2) (layer F.Cu) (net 1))
 (segment (start 66.04 76.2) (end 69.85 76.2) (width 2) (layer F.Cu) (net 1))
 (segment (start 67.31 59.69) (end 66.04 60.96) (width 2) (layer F.Cu) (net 1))
 (segment (start 93.98 71.12) (end 100.33 71.12) (width 2) (layer F.Cu) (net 1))
 (segment (start 67 93.98) (end 69.85 93.98) (width 2) (layer F.Cu) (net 1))
 (segment (start 66.04 93.02) (end 67 93.98) (width 2) (layer F.Cu) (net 1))
 (segment (start 66.04 76.2) (end 66.04 93.02) (width 2) (layer F.Cu) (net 1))
 (segment (start 114.3 50.8) (end 114.3 57.15) (width 2) (layer B.Cu) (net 27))
 (segment (start 111.76 50.8) (end 114.3 50.8) (width 2) (layer B.Cu) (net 27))
 (segment (start 69.85 78.74) (end 71.12 78.74) (width 0.25) (layer F.Cu) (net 23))
 (segment (start 69.85 78.74) (end 77.47 78.74) (width 0.5) (layer F.Cu) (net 23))
 (segment (start 111.76 88.9) (end 118.11 88.9) (width 0.5) (layer F.Cu) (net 4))
 (segment (start 111.76 86.36) (end 118.11 86.36) (width 0.5) (layer F.Cu) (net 5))
 (segment (start 111.76 83.82) (end 118.11 83.82) (width 0.5) (layer F.Cu) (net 6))
 (segment (start 111.76 81.28) (end 118.11 81.28) (width 0.5) (layer F.Cu) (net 7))
 (segment (start 100.13 76.2) (end 100.33 76.2) (width 0.25) (layer B.Cu) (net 24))
 (segment (start 100.33 76.2) (end 100.53 76.2) (width 0.25) (layer B.Cu) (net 24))
 (segment (start 85.09 71.12) (end 85.09 66.04) (width 0.5) (layer B.Cu) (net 24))
 (segment (start 85.09 66.04) (end 87.63 63.5) (width 0.5) (layer B.Cu) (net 24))
 (segment (start 87.63 63.5) (end 92.71 63.5) (width 0.5) (layer B.Cu) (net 24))
 (segment (start 92.71 63.5) (end 91.44 63.5) (width 0.5) (layer B.Cu) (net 24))
 (segment (start 102.87 67.31) (end 102.87 73.86) (width 0.5) (layer B.Cu) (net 24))
 (segment (start 92.71 63.5) (end 99.06 63.5) (width 0.5) (layer B.Cu) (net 24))
 (segment (start 102.87 73.86) (end 100.53 76.2) (width 0.5) (layer B.Cu) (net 24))
 (segment (start 99.06 63.5) (end 102.87 67.31) (width 0.5) (layer B.Cu) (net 24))
 (segment (start 93.98 73.66) (end 85.09 73.66) (width 0.5) (layer F.Cu) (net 28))
 (segment (start 78.74 86.36) (end 81.28 83.82) (width 0.25) (layer B.Cu) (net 22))
 (segment (start 77.47 86.36) (end 78.74 86.36) (width 0.25) (layer B.Cu) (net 22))
 (segment (start 82.55 81.28) (end 81.28 81.28) (width 0.25) (layer B.Cu) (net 21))
 (segment (start 83.82 80.01) (end 82.55 81.28) (width 0.25) (layer B.Cu) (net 21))
 (segment (start 83.82 78.74) (end 81.28 76.2) (width 0.25) (layer B.Cu) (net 21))
 (segment (start 83.82 78.74) (end 83.82 80.01) (width 0.25) (layer B.Cu) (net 21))
 (segment (start 81.28 76.2) (end 77.47 76.2) (width 0.25) (layer B.Cu) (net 21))
 (segment (start 90.14 78.74) (end 91.44 78.74) (width 0.5) (layer B.Cu) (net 20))
 (segment (start 85.09 83.79) (end 85.09 83.82) (width 0.25) (layer B.Cu) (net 20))
 (segment (start 90.14 78.74) (end 87.63 78.74) (width 0.25) (layer B.Cu) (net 20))
 (segment (start 87.63 78.74) (end 85.09 81.28) (width 0.25) (layer B.Cu) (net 20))
 (segment (start 85.09 81.28) (end 85.09 87.63) (width 0.25) (layer B.Cu) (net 20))
 (segment (start 85.09 87.63) (end 82.55 90.17) (width 0.25) (layer B.Cu) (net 20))
 (segment (start 76.2 90.17) (end 72.39 93.98) (width 0.25) (layer B.Cu) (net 20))
 (segment (start 82.55 90.17) (end 76.2 90.17) (width 0.25) (layer B.Cu) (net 20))
 (segment (start 71.12 64.77) (end 74.93 68.58) (width 0.5) (layer B.Cu) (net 16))
 (segment (start 69.85 64.77) (end 71.12 64.77) (width 0.5) (layer B.Cu) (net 16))
 (segment (start 74.93 68.58) (end 77.47 71.12) (width 0.5) (layer B.Cu) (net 16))
 (segment (start 75.97 73.66) (end 77.47 73.66) (width 0.5) (layer B.Cu) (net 17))
 (segment (start 74.93 71.12) (end 74.93 72.62) (width 0.5) (layer B.Cu) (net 17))
 (segment (start 74.93 72.62) (end 75.97 73.66) (width 0.5) (layer B.Cu) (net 17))
 (segment (start 71.12 67.31) (end 74.93 71.12) (width 0.5) (layer B.Cu) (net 17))
 (segment (start 69.85 67.31) (end 71.12 67.31) (width 0.5) (layer B.Cu) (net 17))
 (segment (start 69.85 69.85) (end 71.12 69.85) (width 0.5) (layer B.Cu) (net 18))
 (segment (start 71.12 69.85) (end 73.66 72.39) (width 0.5) (layer B.Cu) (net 18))
 (segment (start 73.66 72.39) (end 73.66 80.01) (width 0.5) (layer B.Cu) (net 18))
 (segment (start 74.93 81.28) (end 77.47 81.28) (width 0.5) (layer B.Cu) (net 18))
 (segment (start 73.66 80.01) (end 74.93 81.28) (width 0.5) (layer B.Cu) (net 18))
 (segment (start 72.39 82.55) (end 73.66 83.82) (width 0.5) (layer B.Cu) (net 19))
 (segment (start 73.66 83.82) (end 77.47 83.82) (width 0.5) (layer B.Cu) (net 19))
 (segment (start 69.85 72.39) (end 71.2 72.39) (width 0.5) (layer B.Cu) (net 19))
 (segment (start 72.39 73.58) (end 72.39 82.55) (width 0.5) (layer B.Cu) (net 19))
 (segment (start 71.2 72.39) (end 72.39 73.58) (width 0.5) (layer B.Cu) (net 19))
 (segment (start 100.33 83.82) (end 104.14 83.82) (width 0.5) (layer F.Cu) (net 14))
 (segment (start 100.33 86.36) (end 104.14 86.36) (width 0.5) (layer F.Cu) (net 15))
 (segment (start 109.22 83.82) (end 106.68 86.36) (width 0.5) (layer F.Cu) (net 12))
 (segment (start 106.68 86.36) (end 106.68 87.63) (width 0.5) (layer F.Cu) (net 12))
 (segment (start 106.68 87.63) (end 104.14 90.17) (width 0.5) (layer F.Cu) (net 12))
 (segment (start 109.22 86.36) (end 106.68 88.9) (width 0.5) (layer F.Cu) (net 2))
 (segment (start 106.68 88.9) (end 106.68 91.44) (width 0.5) (layer F.Cu) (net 2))
 (segment (start 118.03 93.98) (end 119.38 93.98) (width 0.5) (layer F.Cu) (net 1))
 (segment (start 121.92 93.98) (end 121.92 95.25) (width 2) (layer F.Cu) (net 1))
 (segment (start 93.98 96.52) (end 85.09 96.52) (width 2) (layer F.Cu) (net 1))
 (segment (start 118.11 95.25) (end 119.38 96.52) (width 2) (layer F.Cu) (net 1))
 (segment (start 118.11 93.98) (end 118.11 95.25) (width 2) (layer F.Cu) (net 1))
 (segment (start 93.98 96.52) (end 119.38 96.52) (width 2) (layer F.Cu) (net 1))
 (segment (start 119.38 96.52) (end 120.65 96.52) (width 2) (layer F.Cu) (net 1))
 (segment (start 118.11 93.98) (end 121.92 93.98) (width 2) (layer F.Cu) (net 1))
 (segment (start 118.11 93.98) (end 119.38 93.98) (width 2) (layer F.Cu) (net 1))
 (segment (start 119.38 93.98) (end 119.38 95.25) (width 2) (layer F.Cu) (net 1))
 (segment (start 120.65 95.25) (end 121.285 95.885) (width 2) (layer F.Cu) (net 1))
 (segment (start 120.65 96.52) (end 121.285 95.885) (width 2) (layer F.Cu) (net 1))
 (segment (start 119.38 95.25) (end 120.65 95.25) (width 2) (layer F.Cu) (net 1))
 (segment (start 121.285 95.885) (end 121.92 95.25) (width 2) (layer F.Cu) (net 1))
 (segment (start 91.44 86.36) (end 93.98 86.36) (width 2) (layer B.Cu) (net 1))
 (segment (start 91.44 86.36) (end 88.9 86.36) (width 1) (layer B.Cu) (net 1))
 (segment (start 88.9 86.36) (end 81.28 93.98) (width 1) (layer B.Cu) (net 1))
 (segment (start 81.28 93.98) (end 81.28 96.52) (width 1) (layer B.Cu) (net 1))
 (segment (start 81.28 96.52) (end 85.09 96.52) (width 1) (layer B.Cu) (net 1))
 (segment (start 66.04 60.96) (end 69.85 57.15) (width 2) (layer F.Cu) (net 1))
 (segment (start 109.22 81.28) (end 106.68 83.82) (width 0.5) (layer B.Cu) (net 13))
 (segment (start 106.68 83.82) (end 106.68 88.9) (width 0.5) (layer B.Cu) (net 13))
 (segment (start 106.68 88.9) (end 104.14 91.44) (width 0.5) (layer B.Cu) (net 13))
 (segment (start 95.33 93.98) (end 93.98 93.98) (width 0.5) (layer B.Cu) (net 13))
 (segment (start 97.87 91.44) (end 95.33 93.98) (width 0.5) (layer B.Cu) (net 13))
 (segment (start 104.14 91.44) (end 97.87 91.44) (width 0.5) (layer B.Cu) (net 13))
 (segment (start 100.41 93.98) (end 99.06 93.98) (width 0.5) (layer F.Cu) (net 12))
 (segment (start 104.14 90.25) (end 100.41 93.98) (width 0.5) (layer F.Cu) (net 12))
 (segment (start 104.14 90.17) (end 104.14 90.25) (width 0.5) (layer F.Cu) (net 12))
 (segment (start 106.68 91.44) (end 104.14 93.98) (width 0.5) (layer F.Cu) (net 2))
 (segment (start 109.22 88.9) (end 109.22 93.98) (width 0.5) (layer F.Cu) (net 11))
 (segment (start 97.79 74.7) (end 98.83 73.66) (width 0.5) (layer B.Cu) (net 10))
 (segment (start 97.79 88.9) (end 97.79 74.7) (width 0.5) (layer B.Cu) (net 10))
 (segment (start 98.83 73.66) (end 100.33 73.66) (width 0.5) (layer B.Cu) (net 10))
 (segment (start 97.79 88.9) (end 95.25 91.44) (width 0.5) (layer B.Cu) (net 10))
 (segment (start 87.63 91.44) (end 85.09 93.98) (width 0.5) (layer B.Cu) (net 10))
 (segment (start 95.25 91.44) (end 87.63 91.44) (width 0.5) (layer B.Cu) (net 10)))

